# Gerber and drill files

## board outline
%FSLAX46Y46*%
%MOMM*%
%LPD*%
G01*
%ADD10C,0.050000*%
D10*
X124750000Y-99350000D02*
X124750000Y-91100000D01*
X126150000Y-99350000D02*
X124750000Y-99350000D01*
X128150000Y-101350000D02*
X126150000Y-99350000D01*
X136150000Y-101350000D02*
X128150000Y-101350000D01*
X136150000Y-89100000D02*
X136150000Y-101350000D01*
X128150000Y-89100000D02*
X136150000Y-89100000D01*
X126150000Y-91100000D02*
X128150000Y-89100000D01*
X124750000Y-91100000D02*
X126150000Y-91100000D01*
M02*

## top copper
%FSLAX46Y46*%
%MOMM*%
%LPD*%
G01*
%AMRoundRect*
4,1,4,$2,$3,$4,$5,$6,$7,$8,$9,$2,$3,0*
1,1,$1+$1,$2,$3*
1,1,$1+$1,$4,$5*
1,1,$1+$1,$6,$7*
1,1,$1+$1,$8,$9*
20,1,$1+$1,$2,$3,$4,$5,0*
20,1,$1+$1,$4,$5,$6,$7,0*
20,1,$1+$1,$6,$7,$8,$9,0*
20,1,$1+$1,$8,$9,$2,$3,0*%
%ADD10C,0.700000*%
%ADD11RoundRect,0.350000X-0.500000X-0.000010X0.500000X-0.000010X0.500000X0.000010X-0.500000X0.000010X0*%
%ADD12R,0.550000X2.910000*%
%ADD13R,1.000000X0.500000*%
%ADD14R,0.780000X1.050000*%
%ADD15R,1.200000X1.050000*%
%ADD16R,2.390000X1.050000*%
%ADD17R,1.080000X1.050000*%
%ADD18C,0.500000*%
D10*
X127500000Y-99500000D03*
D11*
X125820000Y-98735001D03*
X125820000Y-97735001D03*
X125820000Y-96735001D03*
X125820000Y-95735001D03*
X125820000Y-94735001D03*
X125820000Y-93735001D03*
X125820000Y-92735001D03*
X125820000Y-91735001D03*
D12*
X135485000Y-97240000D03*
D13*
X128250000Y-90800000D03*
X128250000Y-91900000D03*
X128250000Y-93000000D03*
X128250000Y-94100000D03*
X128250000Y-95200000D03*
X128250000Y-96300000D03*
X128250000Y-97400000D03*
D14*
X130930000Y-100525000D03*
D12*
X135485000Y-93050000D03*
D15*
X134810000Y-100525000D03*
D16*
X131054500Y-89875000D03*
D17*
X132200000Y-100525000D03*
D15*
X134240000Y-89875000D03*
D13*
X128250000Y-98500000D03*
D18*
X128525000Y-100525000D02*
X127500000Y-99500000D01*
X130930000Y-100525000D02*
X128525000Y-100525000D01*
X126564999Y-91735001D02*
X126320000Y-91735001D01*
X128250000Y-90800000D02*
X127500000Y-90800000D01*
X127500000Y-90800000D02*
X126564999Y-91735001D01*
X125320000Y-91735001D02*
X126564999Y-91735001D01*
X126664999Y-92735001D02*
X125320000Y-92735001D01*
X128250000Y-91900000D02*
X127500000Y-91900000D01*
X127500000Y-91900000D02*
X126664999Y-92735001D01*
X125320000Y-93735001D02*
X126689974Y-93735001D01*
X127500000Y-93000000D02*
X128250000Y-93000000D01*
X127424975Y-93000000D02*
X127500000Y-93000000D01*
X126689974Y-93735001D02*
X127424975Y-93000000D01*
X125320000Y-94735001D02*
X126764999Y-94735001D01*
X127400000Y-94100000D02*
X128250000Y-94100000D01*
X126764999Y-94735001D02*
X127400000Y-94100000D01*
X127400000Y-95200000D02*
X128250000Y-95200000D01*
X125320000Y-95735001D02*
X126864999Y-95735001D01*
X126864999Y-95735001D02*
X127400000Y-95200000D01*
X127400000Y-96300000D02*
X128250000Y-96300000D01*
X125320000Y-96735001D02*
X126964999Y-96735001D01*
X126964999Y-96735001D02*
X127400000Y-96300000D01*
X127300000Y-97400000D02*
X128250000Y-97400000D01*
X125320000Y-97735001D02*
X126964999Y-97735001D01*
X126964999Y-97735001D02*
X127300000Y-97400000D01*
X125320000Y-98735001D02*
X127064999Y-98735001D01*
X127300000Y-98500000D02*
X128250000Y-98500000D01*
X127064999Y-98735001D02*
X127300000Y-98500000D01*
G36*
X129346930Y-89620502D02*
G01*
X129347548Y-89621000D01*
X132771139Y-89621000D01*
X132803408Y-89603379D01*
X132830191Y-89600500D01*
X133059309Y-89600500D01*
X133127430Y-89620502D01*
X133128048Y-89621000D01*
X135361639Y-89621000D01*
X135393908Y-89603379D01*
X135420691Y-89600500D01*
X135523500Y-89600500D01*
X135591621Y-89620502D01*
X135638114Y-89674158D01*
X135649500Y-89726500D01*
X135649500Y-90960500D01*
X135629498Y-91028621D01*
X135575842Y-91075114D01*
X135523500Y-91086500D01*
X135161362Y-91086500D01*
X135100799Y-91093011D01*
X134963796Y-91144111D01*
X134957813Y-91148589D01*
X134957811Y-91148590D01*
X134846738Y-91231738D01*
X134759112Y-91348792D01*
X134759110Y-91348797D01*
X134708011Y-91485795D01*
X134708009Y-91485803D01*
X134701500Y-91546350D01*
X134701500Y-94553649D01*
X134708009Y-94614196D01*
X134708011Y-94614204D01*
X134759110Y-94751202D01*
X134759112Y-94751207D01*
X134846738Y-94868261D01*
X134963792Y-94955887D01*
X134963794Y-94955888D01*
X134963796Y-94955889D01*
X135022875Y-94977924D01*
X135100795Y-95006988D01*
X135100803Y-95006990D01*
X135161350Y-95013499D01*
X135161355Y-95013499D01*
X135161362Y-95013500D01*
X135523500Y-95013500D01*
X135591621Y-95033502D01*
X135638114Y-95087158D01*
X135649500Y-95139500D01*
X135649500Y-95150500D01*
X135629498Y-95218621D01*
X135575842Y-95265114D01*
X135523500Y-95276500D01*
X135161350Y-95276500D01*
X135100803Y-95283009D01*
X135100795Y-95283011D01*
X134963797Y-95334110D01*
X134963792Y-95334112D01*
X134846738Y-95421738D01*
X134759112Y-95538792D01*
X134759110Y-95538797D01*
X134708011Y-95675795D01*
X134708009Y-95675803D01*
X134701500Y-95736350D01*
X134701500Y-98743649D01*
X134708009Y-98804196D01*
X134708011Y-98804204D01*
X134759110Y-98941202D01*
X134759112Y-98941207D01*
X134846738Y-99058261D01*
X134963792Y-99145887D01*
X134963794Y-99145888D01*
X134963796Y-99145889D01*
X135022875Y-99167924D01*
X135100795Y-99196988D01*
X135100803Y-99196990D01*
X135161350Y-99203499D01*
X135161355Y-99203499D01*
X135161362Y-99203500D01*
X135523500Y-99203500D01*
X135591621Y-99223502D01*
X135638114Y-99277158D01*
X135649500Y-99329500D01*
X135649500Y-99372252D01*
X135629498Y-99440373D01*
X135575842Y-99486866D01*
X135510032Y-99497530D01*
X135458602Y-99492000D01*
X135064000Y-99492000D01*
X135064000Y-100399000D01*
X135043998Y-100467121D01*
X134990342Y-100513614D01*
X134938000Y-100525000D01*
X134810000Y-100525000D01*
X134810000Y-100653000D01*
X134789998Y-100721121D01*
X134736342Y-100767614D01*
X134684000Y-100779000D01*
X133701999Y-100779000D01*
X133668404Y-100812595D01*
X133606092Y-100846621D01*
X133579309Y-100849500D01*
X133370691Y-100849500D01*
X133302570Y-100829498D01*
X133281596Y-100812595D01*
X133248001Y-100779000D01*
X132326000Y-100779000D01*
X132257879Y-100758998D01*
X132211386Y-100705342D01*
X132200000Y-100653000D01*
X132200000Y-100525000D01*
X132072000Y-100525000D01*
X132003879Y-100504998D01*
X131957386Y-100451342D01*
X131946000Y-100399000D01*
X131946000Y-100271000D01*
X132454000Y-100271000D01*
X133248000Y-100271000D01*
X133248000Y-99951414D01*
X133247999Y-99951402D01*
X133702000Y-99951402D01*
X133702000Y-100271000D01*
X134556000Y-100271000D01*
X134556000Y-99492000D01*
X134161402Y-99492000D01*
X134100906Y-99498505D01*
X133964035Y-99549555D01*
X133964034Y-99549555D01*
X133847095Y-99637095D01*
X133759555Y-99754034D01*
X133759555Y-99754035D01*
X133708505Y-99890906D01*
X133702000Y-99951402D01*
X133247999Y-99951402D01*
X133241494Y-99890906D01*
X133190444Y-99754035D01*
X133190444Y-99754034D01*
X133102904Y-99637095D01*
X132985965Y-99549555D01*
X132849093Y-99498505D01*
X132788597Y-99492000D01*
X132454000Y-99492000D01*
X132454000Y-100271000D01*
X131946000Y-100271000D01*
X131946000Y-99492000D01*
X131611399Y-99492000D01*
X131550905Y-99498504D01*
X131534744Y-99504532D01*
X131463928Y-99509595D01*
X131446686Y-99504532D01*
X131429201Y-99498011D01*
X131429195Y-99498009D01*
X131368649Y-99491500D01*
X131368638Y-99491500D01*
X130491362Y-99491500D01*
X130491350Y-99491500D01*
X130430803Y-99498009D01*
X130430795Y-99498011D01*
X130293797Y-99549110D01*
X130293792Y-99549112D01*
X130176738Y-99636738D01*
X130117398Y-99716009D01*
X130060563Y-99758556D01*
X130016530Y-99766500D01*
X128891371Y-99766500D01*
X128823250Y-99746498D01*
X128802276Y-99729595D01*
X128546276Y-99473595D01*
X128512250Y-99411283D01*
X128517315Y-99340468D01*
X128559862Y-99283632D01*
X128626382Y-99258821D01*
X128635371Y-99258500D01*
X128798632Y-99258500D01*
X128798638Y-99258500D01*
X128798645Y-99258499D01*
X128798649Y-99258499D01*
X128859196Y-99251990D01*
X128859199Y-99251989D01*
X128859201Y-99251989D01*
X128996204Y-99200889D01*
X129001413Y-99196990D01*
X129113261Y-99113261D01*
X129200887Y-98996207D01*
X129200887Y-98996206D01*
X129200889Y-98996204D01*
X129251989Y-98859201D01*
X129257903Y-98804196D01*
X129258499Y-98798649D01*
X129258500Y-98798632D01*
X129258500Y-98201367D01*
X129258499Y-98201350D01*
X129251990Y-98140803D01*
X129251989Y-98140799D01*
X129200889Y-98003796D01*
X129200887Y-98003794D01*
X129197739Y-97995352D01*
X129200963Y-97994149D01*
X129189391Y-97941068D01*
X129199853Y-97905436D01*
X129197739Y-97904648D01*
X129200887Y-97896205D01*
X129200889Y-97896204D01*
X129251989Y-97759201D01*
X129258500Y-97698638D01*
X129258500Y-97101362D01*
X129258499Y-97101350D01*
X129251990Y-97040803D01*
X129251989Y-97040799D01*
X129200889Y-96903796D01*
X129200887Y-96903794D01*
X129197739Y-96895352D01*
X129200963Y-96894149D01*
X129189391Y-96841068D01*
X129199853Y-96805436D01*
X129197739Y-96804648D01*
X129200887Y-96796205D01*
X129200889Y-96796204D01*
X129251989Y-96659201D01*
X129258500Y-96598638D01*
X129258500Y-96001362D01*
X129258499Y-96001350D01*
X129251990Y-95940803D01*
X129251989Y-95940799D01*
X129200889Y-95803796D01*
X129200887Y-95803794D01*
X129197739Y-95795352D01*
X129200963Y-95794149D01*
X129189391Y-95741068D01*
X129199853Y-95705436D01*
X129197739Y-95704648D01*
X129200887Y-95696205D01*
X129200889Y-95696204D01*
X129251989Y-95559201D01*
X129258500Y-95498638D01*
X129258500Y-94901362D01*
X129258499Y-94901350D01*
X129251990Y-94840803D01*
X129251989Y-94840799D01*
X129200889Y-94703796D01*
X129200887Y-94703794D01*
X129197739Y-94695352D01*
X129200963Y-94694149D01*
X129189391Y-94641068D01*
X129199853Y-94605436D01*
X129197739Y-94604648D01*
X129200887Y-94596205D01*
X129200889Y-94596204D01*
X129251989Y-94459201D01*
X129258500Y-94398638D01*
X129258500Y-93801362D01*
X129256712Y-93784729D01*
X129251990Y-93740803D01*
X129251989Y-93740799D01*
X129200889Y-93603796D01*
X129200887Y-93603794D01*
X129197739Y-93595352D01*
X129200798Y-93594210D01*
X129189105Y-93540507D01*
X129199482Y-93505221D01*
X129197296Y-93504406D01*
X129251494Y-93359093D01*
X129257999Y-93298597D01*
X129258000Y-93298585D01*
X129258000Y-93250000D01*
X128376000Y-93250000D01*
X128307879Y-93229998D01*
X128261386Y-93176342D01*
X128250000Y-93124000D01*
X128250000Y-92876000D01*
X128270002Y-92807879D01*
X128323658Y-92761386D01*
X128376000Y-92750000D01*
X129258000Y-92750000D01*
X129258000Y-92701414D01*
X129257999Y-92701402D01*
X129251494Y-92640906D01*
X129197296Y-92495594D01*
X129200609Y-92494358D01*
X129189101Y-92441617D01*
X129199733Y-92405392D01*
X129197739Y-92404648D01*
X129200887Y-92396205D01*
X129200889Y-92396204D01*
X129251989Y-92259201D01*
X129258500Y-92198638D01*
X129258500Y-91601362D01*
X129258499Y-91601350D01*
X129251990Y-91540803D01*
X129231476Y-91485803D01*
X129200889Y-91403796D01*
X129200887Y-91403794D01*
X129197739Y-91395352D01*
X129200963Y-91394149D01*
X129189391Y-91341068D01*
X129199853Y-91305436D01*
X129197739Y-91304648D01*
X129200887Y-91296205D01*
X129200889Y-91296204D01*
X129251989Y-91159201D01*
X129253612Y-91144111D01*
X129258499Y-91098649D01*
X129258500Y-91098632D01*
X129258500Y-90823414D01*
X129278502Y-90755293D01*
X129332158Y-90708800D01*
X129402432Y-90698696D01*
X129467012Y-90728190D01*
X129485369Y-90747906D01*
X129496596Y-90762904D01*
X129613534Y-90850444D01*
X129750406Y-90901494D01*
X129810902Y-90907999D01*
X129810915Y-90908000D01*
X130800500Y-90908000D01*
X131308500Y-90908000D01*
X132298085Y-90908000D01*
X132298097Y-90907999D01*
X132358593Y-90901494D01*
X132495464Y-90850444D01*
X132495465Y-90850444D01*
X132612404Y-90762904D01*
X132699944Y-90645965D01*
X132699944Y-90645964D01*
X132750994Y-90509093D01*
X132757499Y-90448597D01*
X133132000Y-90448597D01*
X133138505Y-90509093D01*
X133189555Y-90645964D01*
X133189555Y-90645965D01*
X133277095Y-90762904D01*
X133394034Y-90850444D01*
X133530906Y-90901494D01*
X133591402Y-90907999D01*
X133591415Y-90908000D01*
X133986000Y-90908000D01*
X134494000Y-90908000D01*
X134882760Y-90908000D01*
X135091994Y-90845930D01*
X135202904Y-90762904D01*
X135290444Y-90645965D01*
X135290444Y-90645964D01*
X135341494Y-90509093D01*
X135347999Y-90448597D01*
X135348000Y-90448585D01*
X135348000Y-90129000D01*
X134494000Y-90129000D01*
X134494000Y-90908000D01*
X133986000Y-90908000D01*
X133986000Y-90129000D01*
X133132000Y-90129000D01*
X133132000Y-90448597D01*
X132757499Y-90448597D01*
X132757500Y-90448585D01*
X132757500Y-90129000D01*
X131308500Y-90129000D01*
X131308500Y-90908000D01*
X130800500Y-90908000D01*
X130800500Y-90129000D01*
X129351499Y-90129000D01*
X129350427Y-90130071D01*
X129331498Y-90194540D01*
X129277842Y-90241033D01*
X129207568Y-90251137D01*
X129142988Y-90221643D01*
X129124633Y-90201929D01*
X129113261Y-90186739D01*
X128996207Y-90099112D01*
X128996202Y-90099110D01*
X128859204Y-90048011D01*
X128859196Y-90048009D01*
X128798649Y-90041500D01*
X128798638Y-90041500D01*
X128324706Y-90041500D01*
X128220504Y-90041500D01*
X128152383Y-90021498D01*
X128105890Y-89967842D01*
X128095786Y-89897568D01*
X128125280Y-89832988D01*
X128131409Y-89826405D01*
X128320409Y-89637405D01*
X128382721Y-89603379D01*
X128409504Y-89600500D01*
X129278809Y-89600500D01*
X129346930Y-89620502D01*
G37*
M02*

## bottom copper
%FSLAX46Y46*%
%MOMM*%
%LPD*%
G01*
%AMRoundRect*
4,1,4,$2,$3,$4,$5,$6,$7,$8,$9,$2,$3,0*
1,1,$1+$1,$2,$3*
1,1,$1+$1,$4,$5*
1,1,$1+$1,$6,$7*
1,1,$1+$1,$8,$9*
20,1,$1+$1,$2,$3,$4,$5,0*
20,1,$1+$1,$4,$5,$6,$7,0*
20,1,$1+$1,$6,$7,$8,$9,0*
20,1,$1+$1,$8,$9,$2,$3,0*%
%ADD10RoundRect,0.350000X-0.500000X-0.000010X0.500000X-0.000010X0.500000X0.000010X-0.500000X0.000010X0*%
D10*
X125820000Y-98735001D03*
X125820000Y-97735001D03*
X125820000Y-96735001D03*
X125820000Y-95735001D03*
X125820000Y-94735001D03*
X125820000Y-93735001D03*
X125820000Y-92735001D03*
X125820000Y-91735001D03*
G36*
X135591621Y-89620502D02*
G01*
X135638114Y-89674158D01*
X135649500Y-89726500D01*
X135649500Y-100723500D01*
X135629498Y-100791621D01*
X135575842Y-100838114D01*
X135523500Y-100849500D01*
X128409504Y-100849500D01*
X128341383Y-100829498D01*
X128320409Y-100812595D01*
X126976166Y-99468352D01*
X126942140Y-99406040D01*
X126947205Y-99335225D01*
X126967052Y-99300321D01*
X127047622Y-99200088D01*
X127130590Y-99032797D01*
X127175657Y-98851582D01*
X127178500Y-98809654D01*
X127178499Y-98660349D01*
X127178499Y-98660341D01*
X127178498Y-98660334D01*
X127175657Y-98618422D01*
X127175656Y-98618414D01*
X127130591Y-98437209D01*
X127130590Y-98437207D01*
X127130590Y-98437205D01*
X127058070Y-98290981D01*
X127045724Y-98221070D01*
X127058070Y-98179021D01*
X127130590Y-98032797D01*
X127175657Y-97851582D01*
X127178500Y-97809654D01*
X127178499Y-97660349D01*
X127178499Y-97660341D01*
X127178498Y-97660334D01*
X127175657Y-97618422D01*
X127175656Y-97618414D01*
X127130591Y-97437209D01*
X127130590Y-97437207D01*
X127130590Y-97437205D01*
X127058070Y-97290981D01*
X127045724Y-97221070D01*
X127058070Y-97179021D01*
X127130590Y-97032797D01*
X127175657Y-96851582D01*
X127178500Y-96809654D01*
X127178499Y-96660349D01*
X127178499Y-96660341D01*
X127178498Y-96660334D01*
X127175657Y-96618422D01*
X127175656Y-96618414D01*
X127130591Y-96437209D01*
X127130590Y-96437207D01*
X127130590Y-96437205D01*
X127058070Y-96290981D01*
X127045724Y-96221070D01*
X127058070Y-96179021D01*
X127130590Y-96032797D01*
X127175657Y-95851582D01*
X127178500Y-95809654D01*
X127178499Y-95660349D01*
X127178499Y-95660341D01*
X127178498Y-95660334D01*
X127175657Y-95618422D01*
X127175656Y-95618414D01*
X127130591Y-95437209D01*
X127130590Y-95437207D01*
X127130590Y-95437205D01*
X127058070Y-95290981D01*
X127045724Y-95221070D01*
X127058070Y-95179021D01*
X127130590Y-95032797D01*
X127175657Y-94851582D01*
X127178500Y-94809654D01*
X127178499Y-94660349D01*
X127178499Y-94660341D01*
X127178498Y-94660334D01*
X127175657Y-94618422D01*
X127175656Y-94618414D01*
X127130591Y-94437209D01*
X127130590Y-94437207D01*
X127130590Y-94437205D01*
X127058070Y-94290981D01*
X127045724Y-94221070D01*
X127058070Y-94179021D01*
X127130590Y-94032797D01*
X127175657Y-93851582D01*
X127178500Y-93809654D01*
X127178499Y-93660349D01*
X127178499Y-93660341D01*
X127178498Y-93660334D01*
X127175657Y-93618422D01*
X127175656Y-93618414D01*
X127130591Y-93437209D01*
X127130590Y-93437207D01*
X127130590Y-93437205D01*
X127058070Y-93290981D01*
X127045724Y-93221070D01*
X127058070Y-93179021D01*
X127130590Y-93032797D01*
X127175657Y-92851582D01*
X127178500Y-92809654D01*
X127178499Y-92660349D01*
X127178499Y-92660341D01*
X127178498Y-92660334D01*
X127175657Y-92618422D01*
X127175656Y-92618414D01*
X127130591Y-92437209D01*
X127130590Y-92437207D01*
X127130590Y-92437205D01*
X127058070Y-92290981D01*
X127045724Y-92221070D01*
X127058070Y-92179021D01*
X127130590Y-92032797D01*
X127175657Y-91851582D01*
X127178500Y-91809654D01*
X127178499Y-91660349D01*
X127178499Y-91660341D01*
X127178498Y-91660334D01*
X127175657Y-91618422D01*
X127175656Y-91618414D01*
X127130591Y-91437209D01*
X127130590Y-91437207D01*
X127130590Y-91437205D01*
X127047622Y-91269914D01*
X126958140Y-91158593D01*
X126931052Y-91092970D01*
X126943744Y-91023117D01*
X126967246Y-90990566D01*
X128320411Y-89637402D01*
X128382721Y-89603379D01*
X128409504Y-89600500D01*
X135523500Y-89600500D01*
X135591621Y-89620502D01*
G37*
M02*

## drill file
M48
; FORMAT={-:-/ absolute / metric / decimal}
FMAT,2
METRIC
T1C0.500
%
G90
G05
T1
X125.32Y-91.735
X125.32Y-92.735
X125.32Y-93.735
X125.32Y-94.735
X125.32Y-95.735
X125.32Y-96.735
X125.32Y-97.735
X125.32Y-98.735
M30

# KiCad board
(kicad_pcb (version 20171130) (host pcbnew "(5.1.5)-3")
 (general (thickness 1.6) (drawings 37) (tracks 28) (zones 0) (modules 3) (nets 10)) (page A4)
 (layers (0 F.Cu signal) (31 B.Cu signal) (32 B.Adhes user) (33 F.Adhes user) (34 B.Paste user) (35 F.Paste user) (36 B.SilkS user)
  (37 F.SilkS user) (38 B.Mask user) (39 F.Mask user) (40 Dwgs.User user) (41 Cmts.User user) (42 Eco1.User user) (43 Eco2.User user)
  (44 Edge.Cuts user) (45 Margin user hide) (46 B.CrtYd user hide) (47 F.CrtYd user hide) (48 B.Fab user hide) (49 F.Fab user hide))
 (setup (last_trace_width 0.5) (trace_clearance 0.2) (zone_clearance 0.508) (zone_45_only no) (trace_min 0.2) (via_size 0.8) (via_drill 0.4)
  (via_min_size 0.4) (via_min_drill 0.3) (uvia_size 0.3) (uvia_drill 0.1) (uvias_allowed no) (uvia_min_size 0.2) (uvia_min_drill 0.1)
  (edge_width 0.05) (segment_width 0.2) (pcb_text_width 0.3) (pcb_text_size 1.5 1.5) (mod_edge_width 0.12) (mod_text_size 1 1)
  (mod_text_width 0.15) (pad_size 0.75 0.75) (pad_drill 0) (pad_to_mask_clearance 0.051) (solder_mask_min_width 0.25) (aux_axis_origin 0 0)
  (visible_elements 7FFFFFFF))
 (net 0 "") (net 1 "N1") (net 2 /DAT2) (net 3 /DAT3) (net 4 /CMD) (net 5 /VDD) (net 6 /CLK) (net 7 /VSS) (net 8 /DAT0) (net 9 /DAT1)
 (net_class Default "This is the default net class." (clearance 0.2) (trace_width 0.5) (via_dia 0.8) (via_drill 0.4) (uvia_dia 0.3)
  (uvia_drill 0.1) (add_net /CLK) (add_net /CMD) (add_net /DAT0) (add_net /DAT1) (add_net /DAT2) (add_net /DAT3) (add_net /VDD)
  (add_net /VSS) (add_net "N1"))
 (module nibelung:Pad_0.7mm (layer F.Cu) (at 127.5 99.5)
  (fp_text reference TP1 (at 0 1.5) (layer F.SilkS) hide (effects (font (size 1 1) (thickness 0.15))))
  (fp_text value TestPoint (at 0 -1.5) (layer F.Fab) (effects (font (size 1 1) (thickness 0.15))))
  (pad 1 smd circle (at 0 0) (size 0.7 0.7) (layers F.Cu F.Paste F.Mask) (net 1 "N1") (solder_mask_margin 0.03)))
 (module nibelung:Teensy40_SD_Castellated (layer F.Cu) (at 125.32 91.735001)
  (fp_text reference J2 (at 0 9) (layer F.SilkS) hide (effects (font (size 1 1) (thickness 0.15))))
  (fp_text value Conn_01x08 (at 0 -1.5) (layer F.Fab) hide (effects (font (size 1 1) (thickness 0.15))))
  (pad 8 thru_hole roundrect (at 0 7) (size 1.7 0.7) (drill 0.5 (offset 0.5 0)) (layers *.Cu *.Mask) (roundrect_rratio 0.5) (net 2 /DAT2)
   (solder_mask_margin 0.03))
  (pad 7 thru_hole roundrect (at 0 6) (size 1.7 0.7) (drill 0.5 (offset 0.5 0)) (layers *.Cu *.Mask) (roundrect_rratio 0.5) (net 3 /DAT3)
   (solder_mask_margin 0.03))
  (pad 6 thru_hole roundrect (at 0 5) (size 1.7 0.7) (drill 0.5 (offset 0.5 0)) (layers *.Cu *.Mask) (roundrect_rratio 0.5) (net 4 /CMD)
   (solder_mask_margin 0.03))
  (pad 5 thru_hole roundrect (at 0 4) (size 1.7 0.7) (drill 0.5 (offset 0.5 0)) (layers *.Cu *.Mask) (roundrect_rratio 0.5) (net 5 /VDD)
   (solder_mask_margin 0.03))
  (pad 4 thru_hole roundrect (at 0 3) (size 1.7 0.7) (drill 0.5 (offset 0.5 0)) (layers *.Cu *.Mask) (roundrect_rratio 0.5) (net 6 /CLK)
   (solder_mask_margin 0.03))
  (pad 3 thru_hole roundrect (at 0 2) (size 1.7 0.7) (drill 0.5 (offset 0.5 0)) (layers *.Cu *.Mask) (roundrect_rratio 0.5) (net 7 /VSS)
   (solder_mask_margin 0.03))
  (pad 2 thru_hole roundrect (at 0 1) (size 1.7 0.7) (drill 0.5 (offset 0.5 0)) (layers *.Cu *.Mask) (roundrect_rratio 0.5) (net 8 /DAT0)
   (solder_mask_margin 0.03))
  (pad 1 thru_hole roundrect (at 0 0) (size 1.7 0.7) (drill 0.5 (offset 0.5 0)) (layers *.Cu *.Mask) (roundrect_rratio 0.5) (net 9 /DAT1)
   (solder_mask_margin 0.03)))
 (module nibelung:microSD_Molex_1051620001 (layer F.Cu) (at 127.75 98.75 270)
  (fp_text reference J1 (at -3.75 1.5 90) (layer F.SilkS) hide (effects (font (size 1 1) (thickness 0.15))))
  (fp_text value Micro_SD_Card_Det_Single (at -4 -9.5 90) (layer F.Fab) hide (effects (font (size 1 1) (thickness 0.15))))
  (pad 11 smd rect (at -2.96 -7.46 270) (size 2.91 0.55) (drill (offset 1.45 -0.275)) (layers F.Cu F.Paste F.Mask))
  (pad 8 smd rect (at -7.95 -0.5 270) (size 0.5 1) (layers F.Cu F.Paste F.Mask) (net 9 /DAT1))
  (pad 7 smd rect (at -6.85 -0.5 270) (size 0.5 1) (layers F.Cu F.Paste F.Mask) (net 8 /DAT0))
  (pad 6 smd rect (at -5.75 -0.5 270) (size 0.5 1) (layers F.Cu F.Paste F.Mask) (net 7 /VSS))
  (pad 5 smd rect (at -4.65 -0.5 270) (size 0.5 1) (layers F.Cu F.Paste F.Mask) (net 6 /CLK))
  (pad 4 smd rect (at -3.55 -0.5 270) (size 0.5 1) (layers F.Cu F.Paste F.Mask) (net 5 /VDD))
  (pad 3 smd rect (at -2.45 -0.5 270) (size 0.5 1) (layers F.Cu F.Paste F.Mask) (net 4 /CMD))
  (pad 2 smd rect (at -1.35 -0.5 270) (size 0.5 1) (layers F.Cu F.Paste F.Mask) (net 3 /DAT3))
  (pad 9 smd rect (at 1.775 -3.18 270) (size 1.05 0.78) (layers F.Cu F.Paste F.Mask) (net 1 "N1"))
  (pad 11 smd rect (at -7.15 -7.46 270) (size 2.91 0.55) (drill (offset 1.45 -0.275)) (layers F.Cu F.Paste F.Mask))
  (pad 10 smd rect (at 1.25 -6.46 270) (size 1.05 1.2) (drill (offset 0.525 -0.6)) (layers F.Cu F.Paste F.Mask) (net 7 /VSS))
  (pad 10 smd rect (at -9.4 -2.11 270) (size 1.05 2.39) (drill (offset 0.525 -1.1945)) (layers F.Cu F.Paste F.Mask) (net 7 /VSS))
  (pad 10 smd rect (at 1.25 -3.91 270) (size 1.05 1.08) (drill (offset 0.525 -0.54)) (layers F.Cu F.Paste F.Mask) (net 7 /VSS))
  (pad 10 smd rect (at -9.4 -5.89 270) (size 1.05 1.2) (drill (offset 0.525 -0.6)) (layers F.Cu F.Paste F.Mask) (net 7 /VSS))
  (pad 1 smd rect (at -0.25 -0.5 270) (size 0.5 1) (layers F.Cu F.Paste F.Mask) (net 2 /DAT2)))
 (gr_line (start 124.75 99.35) (end 124.75 91.1) (layer Edge.Cuts) (width 0.05))
 (gr_line (start 126.15 99.35) (end 124.75 99.35) (layer Edge.Cuts) (width 0.05))
 (gr_line (start 128.15 101.35) (end 126.15 99.35) (layer Edge.Cuts) (width 0.05))
 (gr_line (start 136.15 101.35) (end 128.15 101.35) (layer Edge.Cuts) (width 0.05))
 (gr_line (start 136.15 89.1) (end 136.15 101.35) (layer Edge.Cuts) (width 0.05))
 (gr_line (start 128.15 89.1) (end 136.15 89.1) (layer Edge.Cuts) (width 0.05))
 (gr_line (start 126.15 91.1) (end 128.15 89.1) (layer Edge.Cuts) (width 0.05))
 (gr_line (start 124.75 91.1) (end 126.15 91.1) (layer Edge.Cuts) (width 0.05))
 (segment (start 128.525 100.525) (end 127.5 99.5) (width 0.5) (layer F.Cu) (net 1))
 (segment (start 130.93 100.525) (end 128.525 100.525) (width 0.5) (layer F.Cu) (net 1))
 (segment (start 126.564999 91.735001) (end 126.32 91.735001) (width 0.5) (layer F.Cu) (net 9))
 (segment (start 128.25 90.8) (end 127.5 90.8) (width 0.5) (layer F.Cu) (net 9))
 (segment (start 127.5 90.8) (end 126.564999 91.735001) (width 0.5) (layer F.Cu) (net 9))
 (segment (start 125.32 91.735001) (end 126.564999 91.735001) (width 0.5) (layer F.Cu) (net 9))
 (segment (start 126.664999 92.735001) (end 125.32 92.735001) (width 0.5) (layer F.Cu) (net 8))
 (segment (start 128.25 91.9) (end 127.5 91.9) (width 0.5) (layer F.Cu) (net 8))
 (segment (start 127.5 91.9) (end 126.664999 92.735001) (width 0.5) (layer F.Cu) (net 8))
 (segment (start 125.32 93.735001) (end 126.689974 93.735001) (width 0.5) (layer F.Cu) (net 7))
 (segment (start 127.5 93) (end 128.25 93) (width 0.5) (layer F.Cu) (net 7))
 (segment (start 127.424975 93) (end 127.5 93) (width 0.5) (layer F.Cu) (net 7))
 (segment (start 126.689974 93.735001) (end 127.424975 93) (width 0.5) (layer F.Cu) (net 7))
 (segment (start 125.32 94.735001) (end 126.764999 94.735001) (width 0.5) (layer F.Cu) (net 6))
 (segment (start 127.4 94.1) (end 128.25 94.1) (width 0.5) (layer F.Cu) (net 6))
 (segment (start 126.764999 94.735001) (end 127.4 94.1) (width 0.5) (layer F.Cu) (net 6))
 (segment (start 127.4 95.2) (end 128.25 95.2) (width 0.5) (layer F.Cu) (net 5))
 (segment (start 125.32 95.735001) (end 126.864999 95.735001) (width 0.5) (layer F.Cu) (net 5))
 (segment (start 126.864999 95.735001) (end 127.4 95.2) (width 0.5) (layer F.Cu) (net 5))
 (segment (start 127.4 96.3) (end 128.25 96.3) (width 0.5) (layer F.Cu) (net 4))
 (segment (start 125.32 96.735001) (end 126.964999 96.735001) (width 0.5) (layer F.Cu) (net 4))
 (segment (start 126.964999 96.735001) (end 127.4 96.3) (width 0.5) (layer F.Cu) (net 4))
 (segment (start 127.3 97.4) (end 128.25 97.4) (width 0.5) (layer F.Cu) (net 3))
 (segment (start 125.32 97.735001) (end 126.964999 97.735001) (width 0.5) (layer F.Cu) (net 3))
 (segment (start 126.964999 97.735001) (end 127.3 97.4) (width 0.5) (layer F.Cu) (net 3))
 (segment (start 125.32 98.735001) (end 127.064999 98.735001) (width 0.5) (layer F.Cu) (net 2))
 (segment (start 127.3 98.5) (end 128.25 98.5) (width 0.5) (layer F.Cu) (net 2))
 (segment (start 127.064999 98.735001) (end 127.3 98.5) (width 0.5) (layer F.Cu) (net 2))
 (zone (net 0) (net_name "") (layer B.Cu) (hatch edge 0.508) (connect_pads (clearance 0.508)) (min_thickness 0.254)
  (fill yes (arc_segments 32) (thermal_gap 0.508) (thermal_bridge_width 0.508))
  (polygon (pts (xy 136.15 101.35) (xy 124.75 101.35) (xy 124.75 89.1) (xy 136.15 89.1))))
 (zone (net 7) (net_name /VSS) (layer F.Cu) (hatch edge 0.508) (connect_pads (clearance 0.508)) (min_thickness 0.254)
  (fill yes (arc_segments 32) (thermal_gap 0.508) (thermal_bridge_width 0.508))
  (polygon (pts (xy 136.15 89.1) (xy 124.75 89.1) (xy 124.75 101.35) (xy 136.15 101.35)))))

